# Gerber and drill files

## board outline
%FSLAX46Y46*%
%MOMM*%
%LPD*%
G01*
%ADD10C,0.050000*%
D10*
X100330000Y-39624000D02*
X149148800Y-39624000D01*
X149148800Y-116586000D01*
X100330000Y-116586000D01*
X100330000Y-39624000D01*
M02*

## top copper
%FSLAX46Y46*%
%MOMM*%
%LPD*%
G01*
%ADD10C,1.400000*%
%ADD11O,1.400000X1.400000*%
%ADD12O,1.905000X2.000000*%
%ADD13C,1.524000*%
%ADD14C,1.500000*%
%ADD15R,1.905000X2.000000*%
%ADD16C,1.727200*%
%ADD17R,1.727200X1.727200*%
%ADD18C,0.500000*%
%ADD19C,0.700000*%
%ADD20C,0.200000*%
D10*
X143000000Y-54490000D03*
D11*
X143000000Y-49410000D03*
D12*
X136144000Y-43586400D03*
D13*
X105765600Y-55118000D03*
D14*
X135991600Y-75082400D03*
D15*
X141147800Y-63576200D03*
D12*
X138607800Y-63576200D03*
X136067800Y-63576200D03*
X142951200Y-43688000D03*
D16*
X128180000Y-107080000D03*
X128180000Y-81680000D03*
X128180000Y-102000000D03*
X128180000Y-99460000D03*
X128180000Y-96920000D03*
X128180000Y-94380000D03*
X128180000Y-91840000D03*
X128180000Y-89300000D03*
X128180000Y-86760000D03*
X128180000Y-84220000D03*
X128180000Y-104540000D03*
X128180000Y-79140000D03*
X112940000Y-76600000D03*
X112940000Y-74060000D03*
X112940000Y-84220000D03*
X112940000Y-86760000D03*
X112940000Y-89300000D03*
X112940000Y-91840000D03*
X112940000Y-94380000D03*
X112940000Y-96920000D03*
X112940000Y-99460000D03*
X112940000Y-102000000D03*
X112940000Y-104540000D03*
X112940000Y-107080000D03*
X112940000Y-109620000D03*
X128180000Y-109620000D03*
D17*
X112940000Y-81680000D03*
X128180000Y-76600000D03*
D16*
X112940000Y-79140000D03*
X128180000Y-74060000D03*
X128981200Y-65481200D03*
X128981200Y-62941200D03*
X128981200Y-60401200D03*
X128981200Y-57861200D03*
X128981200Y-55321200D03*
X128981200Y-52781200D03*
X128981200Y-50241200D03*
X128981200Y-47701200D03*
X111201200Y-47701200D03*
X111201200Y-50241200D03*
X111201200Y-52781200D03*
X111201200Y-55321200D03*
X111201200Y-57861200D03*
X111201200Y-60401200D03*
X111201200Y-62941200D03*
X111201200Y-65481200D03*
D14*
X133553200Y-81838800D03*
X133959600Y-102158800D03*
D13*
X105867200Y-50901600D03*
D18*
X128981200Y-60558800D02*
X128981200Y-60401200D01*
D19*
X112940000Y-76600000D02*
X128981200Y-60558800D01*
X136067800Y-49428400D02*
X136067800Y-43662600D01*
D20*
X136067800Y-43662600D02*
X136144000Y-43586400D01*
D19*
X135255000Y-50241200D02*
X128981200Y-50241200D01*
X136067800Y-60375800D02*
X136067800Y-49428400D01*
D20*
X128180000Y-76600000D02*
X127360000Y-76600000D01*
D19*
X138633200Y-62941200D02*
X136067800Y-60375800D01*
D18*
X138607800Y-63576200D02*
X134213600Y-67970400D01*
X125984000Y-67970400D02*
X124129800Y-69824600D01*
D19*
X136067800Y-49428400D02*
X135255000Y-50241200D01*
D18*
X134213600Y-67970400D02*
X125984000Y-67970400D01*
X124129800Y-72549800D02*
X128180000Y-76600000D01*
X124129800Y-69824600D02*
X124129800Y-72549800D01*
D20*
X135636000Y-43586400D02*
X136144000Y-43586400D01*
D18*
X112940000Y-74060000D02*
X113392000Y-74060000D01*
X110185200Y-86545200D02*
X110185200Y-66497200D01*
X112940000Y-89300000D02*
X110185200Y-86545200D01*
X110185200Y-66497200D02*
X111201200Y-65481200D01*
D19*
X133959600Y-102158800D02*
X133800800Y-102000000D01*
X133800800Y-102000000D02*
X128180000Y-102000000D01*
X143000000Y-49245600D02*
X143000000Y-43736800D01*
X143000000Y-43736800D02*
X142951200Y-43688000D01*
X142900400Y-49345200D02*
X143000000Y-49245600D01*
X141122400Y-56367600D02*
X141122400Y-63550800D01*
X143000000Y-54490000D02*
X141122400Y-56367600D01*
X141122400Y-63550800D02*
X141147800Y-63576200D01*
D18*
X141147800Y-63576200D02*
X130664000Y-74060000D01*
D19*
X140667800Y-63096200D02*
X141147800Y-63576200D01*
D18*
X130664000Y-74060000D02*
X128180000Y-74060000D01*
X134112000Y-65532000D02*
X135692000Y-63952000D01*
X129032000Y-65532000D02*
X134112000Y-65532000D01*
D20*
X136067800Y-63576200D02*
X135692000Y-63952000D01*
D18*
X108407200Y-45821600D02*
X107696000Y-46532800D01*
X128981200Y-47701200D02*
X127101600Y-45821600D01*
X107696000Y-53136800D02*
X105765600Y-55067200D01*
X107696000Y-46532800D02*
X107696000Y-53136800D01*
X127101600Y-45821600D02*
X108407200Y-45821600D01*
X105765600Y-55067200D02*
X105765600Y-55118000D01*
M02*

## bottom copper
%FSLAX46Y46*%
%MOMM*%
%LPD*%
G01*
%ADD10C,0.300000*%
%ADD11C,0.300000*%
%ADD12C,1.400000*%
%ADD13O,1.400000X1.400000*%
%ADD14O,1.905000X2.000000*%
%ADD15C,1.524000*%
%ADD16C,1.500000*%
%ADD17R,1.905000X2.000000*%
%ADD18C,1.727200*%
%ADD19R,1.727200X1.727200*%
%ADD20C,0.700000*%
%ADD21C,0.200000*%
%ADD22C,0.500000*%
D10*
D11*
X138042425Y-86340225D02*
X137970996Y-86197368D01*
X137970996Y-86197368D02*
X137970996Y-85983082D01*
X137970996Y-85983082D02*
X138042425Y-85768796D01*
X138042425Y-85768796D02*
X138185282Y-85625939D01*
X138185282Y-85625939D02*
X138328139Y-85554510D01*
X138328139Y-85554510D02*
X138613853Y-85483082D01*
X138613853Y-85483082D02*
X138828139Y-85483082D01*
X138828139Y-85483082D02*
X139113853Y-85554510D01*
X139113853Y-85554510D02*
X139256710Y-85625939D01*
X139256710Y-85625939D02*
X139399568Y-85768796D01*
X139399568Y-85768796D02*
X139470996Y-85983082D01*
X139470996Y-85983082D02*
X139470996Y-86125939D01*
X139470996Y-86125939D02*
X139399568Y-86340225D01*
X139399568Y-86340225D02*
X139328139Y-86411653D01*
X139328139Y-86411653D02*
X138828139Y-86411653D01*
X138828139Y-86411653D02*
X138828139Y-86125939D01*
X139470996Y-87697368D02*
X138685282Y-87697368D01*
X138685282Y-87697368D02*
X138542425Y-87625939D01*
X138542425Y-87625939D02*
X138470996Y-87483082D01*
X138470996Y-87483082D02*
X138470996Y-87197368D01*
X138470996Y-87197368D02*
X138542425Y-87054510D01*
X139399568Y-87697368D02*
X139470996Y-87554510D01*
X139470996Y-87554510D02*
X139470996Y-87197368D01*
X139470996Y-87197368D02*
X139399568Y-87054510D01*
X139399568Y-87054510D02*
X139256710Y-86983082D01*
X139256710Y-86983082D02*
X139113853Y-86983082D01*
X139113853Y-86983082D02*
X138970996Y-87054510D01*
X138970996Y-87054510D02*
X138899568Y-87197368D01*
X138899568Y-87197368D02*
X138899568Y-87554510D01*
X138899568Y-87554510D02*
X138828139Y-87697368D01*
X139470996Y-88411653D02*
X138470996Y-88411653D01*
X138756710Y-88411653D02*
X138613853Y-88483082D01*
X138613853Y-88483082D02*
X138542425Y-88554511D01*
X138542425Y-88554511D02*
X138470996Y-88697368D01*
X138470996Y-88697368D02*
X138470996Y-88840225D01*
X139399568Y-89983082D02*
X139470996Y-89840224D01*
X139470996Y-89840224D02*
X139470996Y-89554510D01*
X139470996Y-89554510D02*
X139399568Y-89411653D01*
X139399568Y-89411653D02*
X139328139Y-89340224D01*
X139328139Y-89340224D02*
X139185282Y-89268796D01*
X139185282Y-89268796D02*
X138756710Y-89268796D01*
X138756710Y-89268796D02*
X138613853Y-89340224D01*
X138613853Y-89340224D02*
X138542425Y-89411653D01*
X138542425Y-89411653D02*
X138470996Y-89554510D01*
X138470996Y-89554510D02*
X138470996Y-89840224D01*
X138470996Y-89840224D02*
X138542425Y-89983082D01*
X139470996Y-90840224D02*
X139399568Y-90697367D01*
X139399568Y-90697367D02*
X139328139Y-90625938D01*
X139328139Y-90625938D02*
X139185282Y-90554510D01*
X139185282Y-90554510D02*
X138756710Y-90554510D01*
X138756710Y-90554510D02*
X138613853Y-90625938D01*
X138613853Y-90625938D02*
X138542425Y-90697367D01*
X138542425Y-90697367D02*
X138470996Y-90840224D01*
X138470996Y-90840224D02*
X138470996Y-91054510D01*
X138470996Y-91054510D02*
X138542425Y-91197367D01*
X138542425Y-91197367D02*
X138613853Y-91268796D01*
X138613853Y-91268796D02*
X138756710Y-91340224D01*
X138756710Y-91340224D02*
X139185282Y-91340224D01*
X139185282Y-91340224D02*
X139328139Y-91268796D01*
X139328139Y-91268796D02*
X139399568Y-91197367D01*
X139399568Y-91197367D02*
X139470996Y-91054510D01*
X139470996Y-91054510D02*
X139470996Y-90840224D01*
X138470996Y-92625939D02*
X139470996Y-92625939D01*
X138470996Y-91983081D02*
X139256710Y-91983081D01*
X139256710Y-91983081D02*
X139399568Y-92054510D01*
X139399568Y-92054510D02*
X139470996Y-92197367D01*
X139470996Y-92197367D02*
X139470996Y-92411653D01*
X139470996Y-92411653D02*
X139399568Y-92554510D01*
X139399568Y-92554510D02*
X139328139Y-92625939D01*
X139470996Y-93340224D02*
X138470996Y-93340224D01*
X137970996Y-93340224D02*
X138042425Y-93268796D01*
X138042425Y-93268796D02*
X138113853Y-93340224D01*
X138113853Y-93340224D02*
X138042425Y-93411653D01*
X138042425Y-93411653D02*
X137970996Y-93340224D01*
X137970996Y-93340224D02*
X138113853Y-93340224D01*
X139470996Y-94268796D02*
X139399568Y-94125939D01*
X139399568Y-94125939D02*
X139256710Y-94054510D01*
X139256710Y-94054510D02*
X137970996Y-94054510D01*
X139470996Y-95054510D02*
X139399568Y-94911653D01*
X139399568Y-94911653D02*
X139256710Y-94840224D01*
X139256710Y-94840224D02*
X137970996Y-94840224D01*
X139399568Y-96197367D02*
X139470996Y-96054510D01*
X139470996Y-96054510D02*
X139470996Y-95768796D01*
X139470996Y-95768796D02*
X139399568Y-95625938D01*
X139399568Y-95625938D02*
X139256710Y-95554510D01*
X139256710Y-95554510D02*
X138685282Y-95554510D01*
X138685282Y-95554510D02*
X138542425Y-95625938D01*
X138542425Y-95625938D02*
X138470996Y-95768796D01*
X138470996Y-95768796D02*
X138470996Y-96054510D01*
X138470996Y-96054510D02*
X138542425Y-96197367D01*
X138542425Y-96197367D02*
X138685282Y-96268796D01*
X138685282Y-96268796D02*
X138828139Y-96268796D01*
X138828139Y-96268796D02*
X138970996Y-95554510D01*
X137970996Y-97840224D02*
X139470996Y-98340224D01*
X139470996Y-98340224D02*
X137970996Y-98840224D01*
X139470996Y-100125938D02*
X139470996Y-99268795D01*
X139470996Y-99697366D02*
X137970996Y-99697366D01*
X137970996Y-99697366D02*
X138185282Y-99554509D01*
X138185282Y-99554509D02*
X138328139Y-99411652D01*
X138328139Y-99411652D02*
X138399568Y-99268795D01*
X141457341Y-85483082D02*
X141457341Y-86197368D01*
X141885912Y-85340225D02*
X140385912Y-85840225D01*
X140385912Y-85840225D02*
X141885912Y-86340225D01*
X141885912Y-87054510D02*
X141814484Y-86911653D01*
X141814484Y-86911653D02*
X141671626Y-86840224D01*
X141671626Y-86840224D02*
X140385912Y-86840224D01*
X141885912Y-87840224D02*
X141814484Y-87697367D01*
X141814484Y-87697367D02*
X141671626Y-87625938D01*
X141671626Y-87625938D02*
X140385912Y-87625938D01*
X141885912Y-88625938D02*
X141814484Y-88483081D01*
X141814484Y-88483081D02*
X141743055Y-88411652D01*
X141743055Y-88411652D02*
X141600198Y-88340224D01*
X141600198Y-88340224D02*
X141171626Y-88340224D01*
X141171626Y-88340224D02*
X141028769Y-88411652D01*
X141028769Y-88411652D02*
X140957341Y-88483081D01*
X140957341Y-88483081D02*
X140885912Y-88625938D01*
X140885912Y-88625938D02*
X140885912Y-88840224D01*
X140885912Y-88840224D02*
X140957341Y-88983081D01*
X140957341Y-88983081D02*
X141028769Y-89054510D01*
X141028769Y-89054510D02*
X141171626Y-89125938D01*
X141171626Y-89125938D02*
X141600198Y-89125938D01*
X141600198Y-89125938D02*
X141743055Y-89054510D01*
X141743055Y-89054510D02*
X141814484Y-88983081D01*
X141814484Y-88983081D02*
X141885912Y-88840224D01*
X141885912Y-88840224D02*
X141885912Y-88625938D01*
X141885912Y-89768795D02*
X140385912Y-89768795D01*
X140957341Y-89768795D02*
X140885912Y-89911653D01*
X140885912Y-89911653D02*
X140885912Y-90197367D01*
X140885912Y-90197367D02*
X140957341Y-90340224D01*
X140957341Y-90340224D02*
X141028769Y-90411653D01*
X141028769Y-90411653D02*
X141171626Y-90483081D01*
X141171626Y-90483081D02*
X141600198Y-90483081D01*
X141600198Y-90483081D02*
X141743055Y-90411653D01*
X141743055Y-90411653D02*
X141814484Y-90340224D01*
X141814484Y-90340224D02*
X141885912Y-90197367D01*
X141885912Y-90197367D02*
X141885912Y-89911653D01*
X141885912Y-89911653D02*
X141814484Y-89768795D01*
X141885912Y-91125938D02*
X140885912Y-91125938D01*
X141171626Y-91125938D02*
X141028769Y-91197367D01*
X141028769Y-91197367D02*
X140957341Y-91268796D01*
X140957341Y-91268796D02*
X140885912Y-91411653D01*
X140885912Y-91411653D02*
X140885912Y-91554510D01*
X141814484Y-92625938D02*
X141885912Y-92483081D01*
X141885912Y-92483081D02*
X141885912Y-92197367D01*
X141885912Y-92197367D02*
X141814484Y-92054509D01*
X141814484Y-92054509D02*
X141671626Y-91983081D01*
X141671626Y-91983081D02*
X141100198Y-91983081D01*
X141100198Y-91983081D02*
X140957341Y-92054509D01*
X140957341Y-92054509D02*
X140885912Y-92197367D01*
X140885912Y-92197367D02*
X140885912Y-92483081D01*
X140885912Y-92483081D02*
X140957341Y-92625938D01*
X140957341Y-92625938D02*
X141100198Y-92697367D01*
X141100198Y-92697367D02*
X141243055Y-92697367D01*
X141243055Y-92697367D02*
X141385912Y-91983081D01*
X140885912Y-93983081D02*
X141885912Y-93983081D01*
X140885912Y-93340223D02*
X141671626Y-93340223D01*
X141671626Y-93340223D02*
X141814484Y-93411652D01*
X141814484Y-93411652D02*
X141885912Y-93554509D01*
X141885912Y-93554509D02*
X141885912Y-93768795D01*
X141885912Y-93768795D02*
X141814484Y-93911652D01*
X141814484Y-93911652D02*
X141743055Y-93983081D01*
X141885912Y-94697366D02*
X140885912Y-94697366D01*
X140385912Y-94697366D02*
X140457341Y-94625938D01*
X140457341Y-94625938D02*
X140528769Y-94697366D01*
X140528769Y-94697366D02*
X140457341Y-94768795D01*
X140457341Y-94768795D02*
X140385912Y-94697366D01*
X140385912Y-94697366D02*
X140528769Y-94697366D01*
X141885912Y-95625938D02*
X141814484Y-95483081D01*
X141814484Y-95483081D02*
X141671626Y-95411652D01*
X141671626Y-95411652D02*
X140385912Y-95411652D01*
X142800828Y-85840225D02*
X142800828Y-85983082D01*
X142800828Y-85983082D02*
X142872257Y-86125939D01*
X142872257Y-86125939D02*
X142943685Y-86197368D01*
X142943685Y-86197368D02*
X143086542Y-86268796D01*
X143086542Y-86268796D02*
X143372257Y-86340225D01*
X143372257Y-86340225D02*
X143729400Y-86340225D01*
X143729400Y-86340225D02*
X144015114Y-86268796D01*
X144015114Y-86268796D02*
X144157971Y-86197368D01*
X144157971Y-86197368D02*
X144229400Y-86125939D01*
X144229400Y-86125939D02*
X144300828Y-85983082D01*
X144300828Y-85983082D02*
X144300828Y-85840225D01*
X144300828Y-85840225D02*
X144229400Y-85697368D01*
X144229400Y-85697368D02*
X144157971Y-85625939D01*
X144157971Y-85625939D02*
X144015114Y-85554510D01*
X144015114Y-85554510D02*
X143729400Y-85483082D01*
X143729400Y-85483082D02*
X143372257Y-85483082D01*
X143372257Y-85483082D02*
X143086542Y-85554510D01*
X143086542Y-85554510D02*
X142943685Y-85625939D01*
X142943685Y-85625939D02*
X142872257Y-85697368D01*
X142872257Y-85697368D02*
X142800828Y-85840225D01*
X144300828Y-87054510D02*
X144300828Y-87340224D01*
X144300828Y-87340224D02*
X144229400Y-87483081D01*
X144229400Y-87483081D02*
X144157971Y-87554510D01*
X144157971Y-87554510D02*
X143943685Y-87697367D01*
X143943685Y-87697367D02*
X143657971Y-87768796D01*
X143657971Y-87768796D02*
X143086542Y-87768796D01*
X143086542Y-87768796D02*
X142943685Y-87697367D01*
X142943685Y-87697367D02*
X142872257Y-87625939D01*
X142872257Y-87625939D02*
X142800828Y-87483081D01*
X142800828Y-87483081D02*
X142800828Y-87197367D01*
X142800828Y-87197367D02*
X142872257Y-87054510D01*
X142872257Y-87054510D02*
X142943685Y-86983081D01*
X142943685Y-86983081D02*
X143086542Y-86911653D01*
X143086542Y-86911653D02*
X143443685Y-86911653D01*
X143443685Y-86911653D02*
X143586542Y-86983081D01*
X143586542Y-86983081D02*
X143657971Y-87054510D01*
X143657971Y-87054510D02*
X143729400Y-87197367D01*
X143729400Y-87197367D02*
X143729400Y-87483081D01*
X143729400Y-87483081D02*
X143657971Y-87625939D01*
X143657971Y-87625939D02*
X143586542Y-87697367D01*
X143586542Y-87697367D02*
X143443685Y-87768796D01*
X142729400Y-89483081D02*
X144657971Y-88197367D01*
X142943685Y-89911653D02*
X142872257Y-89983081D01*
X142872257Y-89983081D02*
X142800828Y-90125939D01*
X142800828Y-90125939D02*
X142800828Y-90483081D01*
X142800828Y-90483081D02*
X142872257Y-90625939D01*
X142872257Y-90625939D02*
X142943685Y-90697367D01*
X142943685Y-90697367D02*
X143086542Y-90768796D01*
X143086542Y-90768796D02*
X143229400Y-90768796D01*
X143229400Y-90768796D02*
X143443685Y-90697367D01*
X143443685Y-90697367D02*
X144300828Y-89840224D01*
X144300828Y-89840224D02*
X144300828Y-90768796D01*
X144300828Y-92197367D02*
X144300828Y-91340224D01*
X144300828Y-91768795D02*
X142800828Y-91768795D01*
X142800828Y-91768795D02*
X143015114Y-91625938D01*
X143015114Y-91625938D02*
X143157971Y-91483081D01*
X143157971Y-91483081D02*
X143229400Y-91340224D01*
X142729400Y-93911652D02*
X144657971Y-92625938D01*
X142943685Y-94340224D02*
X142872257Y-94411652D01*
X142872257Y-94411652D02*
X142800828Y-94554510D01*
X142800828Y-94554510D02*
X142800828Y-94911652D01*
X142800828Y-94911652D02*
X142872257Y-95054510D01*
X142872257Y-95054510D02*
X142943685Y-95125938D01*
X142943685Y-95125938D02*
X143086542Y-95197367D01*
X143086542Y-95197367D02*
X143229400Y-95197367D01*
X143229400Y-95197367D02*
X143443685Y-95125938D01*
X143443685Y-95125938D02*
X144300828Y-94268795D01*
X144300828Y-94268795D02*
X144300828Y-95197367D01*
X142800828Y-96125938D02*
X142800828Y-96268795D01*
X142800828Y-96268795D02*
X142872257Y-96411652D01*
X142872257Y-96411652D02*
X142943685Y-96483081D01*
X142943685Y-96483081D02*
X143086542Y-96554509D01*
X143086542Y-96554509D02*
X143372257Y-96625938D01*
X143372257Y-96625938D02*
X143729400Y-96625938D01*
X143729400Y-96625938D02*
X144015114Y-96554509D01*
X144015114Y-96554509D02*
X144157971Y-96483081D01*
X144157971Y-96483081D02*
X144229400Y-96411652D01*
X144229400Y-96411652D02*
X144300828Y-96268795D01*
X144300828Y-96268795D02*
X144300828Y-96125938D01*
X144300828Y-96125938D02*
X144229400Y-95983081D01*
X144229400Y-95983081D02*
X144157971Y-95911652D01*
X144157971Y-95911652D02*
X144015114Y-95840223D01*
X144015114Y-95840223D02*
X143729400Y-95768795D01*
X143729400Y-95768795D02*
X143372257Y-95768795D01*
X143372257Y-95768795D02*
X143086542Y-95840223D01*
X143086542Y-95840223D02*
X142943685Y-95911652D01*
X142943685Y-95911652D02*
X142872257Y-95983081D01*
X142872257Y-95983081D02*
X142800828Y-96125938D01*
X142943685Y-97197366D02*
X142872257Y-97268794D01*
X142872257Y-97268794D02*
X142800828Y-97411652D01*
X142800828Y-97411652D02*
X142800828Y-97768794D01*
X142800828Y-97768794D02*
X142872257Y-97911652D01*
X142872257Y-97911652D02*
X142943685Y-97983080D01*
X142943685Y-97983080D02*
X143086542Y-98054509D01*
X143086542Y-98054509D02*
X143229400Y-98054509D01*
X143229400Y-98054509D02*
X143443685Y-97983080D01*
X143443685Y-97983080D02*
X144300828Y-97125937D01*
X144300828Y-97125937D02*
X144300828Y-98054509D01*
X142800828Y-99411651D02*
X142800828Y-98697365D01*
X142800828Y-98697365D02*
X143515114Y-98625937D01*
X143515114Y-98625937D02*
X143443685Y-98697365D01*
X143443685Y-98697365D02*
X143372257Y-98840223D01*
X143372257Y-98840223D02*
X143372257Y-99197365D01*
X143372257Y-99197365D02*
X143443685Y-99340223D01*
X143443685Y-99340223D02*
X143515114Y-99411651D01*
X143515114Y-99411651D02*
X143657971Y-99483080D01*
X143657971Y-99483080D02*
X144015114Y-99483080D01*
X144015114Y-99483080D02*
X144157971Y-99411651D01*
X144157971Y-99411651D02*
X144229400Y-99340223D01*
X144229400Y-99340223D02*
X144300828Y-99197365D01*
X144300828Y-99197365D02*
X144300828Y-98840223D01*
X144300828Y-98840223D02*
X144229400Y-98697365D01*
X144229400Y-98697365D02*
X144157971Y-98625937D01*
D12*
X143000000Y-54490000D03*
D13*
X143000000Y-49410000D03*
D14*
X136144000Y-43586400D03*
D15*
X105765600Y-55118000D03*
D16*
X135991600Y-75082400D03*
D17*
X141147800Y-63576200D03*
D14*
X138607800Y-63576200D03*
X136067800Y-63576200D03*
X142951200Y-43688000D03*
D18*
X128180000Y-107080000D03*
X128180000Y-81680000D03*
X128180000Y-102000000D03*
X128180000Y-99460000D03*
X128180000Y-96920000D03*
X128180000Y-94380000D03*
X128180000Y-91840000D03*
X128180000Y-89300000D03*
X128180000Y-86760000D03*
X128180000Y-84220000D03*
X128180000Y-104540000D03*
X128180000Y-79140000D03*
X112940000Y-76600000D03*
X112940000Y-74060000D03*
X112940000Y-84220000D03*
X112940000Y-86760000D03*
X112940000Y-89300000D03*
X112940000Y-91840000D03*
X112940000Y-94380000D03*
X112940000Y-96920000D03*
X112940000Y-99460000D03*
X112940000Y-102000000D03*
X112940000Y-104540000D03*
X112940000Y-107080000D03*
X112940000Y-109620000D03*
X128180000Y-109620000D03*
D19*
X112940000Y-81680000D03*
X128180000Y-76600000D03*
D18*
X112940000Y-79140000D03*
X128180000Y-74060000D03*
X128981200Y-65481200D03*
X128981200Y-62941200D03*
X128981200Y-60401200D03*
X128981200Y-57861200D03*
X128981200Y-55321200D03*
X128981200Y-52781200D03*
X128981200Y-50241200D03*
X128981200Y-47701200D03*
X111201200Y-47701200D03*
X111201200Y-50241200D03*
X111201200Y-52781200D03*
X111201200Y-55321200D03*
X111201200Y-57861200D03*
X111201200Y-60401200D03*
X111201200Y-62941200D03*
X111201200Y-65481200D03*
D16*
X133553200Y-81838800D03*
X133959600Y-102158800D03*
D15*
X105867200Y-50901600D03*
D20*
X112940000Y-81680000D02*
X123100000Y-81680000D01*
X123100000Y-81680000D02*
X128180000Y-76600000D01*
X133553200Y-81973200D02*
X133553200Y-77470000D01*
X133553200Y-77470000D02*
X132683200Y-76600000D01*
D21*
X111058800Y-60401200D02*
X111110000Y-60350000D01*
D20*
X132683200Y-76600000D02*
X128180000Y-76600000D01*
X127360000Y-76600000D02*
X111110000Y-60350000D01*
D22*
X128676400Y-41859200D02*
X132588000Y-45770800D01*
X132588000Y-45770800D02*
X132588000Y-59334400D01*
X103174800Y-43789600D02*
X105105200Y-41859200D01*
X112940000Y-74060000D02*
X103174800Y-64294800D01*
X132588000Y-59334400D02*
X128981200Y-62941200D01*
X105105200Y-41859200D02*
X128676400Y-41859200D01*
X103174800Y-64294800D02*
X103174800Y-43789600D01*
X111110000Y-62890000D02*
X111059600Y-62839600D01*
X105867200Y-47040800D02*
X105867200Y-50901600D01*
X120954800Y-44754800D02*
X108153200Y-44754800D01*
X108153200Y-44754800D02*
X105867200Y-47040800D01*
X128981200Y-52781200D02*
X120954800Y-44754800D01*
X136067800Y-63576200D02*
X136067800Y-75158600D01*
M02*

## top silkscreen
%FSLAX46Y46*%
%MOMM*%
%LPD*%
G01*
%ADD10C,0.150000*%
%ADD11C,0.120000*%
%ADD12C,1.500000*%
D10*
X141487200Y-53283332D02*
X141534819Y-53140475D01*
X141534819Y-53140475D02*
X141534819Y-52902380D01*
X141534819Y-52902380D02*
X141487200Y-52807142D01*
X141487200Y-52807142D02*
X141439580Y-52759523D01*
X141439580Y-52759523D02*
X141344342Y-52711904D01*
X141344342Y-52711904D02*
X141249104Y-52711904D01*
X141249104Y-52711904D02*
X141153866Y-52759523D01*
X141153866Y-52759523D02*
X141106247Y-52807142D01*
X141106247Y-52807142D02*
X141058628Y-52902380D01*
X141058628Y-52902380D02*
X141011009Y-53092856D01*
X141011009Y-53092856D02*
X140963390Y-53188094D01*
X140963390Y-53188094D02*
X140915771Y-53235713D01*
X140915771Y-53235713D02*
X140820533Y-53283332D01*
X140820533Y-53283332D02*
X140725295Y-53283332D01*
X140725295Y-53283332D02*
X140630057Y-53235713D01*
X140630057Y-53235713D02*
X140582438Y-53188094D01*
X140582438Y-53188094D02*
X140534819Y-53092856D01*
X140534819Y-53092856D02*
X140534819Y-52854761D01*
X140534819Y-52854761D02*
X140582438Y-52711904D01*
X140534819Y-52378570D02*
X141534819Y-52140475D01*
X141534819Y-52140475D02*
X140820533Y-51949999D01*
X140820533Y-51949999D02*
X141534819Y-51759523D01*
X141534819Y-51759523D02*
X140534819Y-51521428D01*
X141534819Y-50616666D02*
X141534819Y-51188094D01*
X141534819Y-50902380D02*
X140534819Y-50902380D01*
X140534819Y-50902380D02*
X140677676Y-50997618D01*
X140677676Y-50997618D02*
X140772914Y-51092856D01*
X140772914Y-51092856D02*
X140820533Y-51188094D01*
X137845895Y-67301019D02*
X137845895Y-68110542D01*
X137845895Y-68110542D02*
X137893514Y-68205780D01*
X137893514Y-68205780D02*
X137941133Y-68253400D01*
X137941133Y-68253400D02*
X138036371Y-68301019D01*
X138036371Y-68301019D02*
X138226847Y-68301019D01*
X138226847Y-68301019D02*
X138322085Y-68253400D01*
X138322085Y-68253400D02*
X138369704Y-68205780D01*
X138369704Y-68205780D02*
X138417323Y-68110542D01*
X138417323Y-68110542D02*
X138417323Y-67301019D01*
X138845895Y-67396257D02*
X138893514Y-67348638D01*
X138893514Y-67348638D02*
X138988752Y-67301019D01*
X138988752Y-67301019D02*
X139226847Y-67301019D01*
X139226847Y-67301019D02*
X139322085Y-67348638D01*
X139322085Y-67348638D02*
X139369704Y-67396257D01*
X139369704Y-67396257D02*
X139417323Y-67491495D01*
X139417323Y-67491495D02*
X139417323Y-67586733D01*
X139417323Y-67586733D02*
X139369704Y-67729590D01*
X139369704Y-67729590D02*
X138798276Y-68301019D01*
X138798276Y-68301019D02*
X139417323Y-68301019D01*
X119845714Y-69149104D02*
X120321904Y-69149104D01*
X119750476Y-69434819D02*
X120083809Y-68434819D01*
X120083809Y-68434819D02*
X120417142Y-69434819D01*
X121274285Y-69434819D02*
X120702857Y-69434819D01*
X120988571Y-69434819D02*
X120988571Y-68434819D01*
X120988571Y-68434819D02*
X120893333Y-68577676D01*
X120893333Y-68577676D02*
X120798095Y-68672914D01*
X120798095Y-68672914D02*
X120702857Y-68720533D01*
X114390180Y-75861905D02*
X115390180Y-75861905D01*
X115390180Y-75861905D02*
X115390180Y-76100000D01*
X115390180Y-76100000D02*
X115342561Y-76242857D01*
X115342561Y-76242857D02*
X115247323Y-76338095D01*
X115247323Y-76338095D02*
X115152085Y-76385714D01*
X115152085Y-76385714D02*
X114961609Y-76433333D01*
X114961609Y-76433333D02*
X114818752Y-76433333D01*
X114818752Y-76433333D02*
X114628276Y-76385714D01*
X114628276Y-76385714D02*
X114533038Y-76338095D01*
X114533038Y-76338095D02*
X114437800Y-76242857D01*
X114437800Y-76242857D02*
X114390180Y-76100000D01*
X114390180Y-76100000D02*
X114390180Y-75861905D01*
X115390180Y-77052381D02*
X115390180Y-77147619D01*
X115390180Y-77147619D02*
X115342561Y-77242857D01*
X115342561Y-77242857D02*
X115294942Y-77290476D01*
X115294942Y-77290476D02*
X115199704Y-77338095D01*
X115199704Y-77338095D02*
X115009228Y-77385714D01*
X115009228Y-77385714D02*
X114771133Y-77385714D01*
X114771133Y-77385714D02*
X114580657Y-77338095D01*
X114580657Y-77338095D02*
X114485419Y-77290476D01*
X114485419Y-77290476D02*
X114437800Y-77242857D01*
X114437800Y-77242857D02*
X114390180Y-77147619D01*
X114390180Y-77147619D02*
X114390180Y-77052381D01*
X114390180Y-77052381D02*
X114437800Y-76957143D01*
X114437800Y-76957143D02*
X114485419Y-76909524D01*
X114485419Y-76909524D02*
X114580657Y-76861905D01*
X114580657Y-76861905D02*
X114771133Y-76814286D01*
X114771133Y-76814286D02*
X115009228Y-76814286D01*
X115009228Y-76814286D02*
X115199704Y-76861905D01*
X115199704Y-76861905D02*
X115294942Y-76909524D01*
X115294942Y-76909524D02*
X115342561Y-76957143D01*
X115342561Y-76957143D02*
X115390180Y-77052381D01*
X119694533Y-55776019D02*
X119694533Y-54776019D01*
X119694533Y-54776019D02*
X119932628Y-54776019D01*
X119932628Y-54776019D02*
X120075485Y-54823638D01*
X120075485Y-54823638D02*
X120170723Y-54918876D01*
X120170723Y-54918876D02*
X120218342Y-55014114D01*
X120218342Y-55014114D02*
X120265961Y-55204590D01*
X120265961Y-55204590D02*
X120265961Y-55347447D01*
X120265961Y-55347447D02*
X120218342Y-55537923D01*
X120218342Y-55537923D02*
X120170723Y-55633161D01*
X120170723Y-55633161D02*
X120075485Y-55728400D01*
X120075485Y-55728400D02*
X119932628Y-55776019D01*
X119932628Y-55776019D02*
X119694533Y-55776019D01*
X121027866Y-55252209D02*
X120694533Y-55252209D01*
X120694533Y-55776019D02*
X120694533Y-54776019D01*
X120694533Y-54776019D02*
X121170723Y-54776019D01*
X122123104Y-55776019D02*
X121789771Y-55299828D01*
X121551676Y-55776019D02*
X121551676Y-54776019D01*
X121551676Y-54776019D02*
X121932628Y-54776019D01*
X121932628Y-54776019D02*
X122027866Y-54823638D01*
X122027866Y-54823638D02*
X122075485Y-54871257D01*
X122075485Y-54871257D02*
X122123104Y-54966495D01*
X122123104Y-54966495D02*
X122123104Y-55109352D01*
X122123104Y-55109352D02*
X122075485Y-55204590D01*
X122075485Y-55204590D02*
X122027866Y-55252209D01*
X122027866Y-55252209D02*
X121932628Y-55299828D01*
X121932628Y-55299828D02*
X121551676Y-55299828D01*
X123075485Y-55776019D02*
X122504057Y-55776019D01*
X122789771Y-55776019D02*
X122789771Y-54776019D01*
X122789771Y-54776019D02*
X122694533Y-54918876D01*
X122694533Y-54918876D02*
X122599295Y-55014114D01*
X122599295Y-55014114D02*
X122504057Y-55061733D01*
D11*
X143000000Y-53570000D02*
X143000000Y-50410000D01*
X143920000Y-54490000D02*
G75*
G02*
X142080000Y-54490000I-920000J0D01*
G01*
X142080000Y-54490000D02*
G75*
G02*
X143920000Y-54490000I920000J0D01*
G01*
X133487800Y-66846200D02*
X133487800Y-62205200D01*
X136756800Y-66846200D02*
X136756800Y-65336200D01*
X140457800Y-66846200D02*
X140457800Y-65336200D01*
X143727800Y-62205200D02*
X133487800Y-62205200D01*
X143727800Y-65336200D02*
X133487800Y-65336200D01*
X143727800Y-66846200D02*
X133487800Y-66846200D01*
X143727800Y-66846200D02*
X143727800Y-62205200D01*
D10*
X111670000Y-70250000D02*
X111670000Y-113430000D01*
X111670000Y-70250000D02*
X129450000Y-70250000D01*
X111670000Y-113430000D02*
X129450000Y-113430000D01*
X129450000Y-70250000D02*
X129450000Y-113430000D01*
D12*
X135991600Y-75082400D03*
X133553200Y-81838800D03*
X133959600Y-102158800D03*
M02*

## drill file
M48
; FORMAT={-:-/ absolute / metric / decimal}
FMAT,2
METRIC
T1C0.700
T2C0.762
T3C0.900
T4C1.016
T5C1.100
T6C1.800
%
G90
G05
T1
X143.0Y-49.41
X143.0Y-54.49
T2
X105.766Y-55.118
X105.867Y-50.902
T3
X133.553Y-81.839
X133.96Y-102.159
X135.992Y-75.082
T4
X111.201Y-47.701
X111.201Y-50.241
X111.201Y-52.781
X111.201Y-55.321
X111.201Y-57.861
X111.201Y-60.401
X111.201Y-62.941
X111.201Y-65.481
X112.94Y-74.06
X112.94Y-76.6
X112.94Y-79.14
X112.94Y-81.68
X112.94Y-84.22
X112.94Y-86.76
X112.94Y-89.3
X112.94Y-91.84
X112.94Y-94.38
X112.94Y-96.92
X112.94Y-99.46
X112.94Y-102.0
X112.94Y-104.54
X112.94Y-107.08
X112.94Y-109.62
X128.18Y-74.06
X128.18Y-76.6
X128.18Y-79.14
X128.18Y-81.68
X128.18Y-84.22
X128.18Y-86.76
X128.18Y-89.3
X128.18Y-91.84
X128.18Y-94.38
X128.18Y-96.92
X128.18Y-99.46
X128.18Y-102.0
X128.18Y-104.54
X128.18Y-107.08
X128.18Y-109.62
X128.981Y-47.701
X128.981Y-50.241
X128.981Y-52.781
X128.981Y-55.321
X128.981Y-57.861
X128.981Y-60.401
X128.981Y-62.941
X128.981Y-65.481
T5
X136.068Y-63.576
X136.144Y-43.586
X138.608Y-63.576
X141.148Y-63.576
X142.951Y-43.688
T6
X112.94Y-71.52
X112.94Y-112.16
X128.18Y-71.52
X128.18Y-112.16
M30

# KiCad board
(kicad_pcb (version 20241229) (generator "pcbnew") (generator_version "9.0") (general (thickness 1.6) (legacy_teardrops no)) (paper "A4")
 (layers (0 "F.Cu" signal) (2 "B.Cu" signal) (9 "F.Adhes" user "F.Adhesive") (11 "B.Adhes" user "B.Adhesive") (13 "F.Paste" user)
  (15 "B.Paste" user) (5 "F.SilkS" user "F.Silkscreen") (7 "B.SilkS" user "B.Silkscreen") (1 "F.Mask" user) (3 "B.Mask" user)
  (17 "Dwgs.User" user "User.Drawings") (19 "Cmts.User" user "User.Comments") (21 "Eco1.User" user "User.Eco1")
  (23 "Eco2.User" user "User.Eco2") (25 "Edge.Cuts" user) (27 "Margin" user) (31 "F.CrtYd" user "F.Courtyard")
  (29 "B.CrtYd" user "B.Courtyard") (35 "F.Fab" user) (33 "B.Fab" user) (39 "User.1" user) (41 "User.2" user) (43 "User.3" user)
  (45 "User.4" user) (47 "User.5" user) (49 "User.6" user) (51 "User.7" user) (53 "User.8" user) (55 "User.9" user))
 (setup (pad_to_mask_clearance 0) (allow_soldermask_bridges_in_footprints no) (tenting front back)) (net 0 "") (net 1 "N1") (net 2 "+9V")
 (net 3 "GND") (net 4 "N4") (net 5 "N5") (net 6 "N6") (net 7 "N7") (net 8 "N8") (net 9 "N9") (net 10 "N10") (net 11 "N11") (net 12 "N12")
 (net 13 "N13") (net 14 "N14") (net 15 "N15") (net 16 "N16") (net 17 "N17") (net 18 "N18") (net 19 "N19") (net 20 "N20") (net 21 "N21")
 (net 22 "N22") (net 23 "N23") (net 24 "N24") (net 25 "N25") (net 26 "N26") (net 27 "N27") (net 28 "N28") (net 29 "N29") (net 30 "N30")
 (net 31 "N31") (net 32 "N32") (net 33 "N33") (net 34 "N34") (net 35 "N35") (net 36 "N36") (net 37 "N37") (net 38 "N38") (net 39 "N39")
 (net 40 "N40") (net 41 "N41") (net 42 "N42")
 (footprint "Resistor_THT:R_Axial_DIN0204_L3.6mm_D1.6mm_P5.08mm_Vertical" (layer "F.Cu") (at 143 54.49 90)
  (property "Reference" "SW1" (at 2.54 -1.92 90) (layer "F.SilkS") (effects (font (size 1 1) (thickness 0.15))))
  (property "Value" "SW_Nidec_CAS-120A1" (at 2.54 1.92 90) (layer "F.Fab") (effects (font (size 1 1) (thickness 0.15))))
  (fp_line (start 0.92 0) (end 4.08 0) (stroke (width 0.12) (type solid)) (layer "F.SilkS"))
  (fp_circle (center 0 0) (end 0.92 0) (stroke (width 0.12) (type solid)) (fill no) (layer "F.SilkS"))
  (pad "1" thru_hole circle (at 0 0 90) (size 1.4 1.4) (drill 0.7) (layers "*.Cu" "*.Mask") (remove_unused_layers no) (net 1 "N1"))
  (pad "2" thru_hole oval (at 5.08 0 90) (size 1.4 1.4) (drill 0.7) (layers "*.Cu" "*.Mask") (remove_unused_layers no) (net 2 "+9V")))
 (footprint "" (layer "F.Cu") (at 136.144 43.5864)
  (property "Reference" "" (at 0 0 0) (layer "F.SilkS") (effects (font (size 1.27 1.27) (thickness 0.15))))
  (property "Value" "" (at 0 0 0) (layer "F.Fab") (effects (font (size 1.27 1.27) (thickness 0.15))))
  (pad "3" thru_hole oval (at 0 0 180) (size 1.905 2) (drill 1.1) (layers "*.Cu" "*.Mask") (remove_unused_layers no) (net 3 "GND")))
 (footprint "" (layer "F.Cu") (at 105.7656 55.118)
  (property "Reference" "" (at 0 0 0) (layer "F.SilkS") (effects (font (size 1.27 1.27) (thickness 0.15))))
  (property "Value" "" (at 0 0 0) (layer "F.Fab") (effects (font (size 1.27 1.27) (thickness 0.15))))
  (pad "8" thru_hole circle (at 0 0) (size 1.524 1.524) (drill 0.762) (layers "*.Cu" "*.Mask") (remove_unused_layers no) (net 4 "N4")))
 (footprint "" (layer "F.Cu") (at 135.9916 75.0824)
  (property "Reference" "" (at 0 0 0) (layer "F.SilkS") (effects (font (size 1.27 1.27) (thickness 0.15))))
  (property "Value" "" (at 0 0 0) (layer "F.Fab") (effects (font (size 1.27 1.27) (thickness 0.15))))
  (pad "3" thru_hole circle (at 0 0 90) (size 1.5 1.5) (drill 0.9) (layers "*.Cu" "*.Mask" "F.SilkS") (remove_unused_layers no) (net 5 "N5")))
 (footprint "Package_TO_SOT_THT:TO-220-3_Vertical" (layer "F.Cu") (at 141.1478 63.5762 180)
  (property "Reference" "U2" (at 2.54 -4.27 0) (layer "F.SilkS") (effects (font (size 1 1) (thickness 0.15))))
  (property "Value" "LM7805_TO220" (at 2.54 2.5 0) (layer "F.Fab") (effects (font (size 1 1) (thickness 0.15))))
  (fp_line (start 7.66 -3.27) (end 7.66 1.371) (stroke (width 0.12) (type solid)) (layer "F.SilkS"))
  (fp_line (start 4.391 -3.27) (end 4.391 -1.76) (stroke (width 0.12) (type solid)) (layer "F.SilkS"))
  (fp_line (start 0.69 -3.27) (end 0.69 -1.76) (stroke (width 0.12) (type solid)) (layer "F.SilkS"))
  (fp_line (start -2.58 1.371) (end 7.66 1.371) (stroke (width 0.12) (type solid)) (layer "F.SilkS"))
  (fp_line (start -2.58 -1.76) (end 7.66 -1.76) (stroke (width 0.12) (type solid)) (layer "F.SilkS"))
  (fp_line (start -2.58 -3.27) (end 7.66 -3.27) (stroke (width 0.12) (type solid)) (layer "F.SilkS"))
  (fp_line (start -2.58 -3.27) (end -2.58 1.371) (stroke (width 0.12) (type solid)) (layer "F.SilkS"))
  (pad "1" thru_hole rect (at 0 0 180) (size 1.905 2) (drill 1.1) (layers "*.Cu" "*.Mask") (remove_unused_layers no) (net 1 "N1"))
  (pad "2" thru_hole oval (at 2.54 0 180) (size 1.905 2) (drill 1.1) (layers "*.Cu" "*.Mask") (remove_unused_layers no) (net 3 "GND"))
  (pad "3" thru_hole oval (at 5.08 0 180) (size 1.905 2) (drill 1.1) (layers "*.Cu" "*.Mask") (remove_unused_layers no) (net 5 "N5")))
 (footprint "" (layer "F.Cu") (at 142.9512 43.688)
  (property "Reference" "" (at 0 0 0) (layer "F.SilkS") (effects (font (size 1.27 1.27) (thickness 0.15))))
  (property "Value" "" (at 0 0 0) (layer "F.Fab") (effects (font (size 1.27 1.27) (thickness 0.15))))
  (pad "3" thru_hole oval (at 0 0 180) (size 1.905 2) (drill 1.1) (layers "*.Cu" "*.Mask") (remove_unused_layers no) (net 2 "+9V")))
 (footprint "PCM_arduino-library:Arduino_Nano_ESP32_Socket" (layer "F.Cu") (at 120.56 113.43)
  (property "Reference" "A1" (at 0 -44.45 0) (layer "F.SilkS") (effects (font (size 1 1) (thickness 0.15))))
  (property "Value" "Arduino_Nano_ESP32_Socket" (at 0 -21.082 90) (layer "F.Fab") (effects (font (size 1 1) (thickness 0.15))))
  (fp_line (start -8.89 -43.18) (end -8.89 0) (stroke (width 0.15) (type solid)) (layer "F.SilkS"))
  (fp_line (start -8.89 -43.18) (end 8.89 -43.18) (stroke (width 0.15) (type solid)) (layer "F.SilkS"))
  (fp_line (start -8.89 0) (end 8.89 0) (stroke (width 0.15) (type solid)) (layer "F.SilkS"))
  (fp_line (start 8.89 -43.18) (end 8.89 0) (stroke (width 0.15) (type solid)) (layer "F.SilkS"))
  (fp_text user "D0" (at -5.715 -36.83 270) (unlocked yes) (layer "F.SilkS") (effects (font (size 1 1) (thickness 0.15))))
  (pad "" np_thru_hole circle (at -7.62 -41.91) (size 1.8 1.8) (drill 1.8) (layers "*.Cu" "*.Mask"))
  (pad "" np_thru_hole circle (at -7.62 -1.27) (size 1.8 1.8) (drill 1.8) (layers "*.Cu" "*.Mask"))
  (pad "" np_thru_hole circle (at 7.62 -41.91) (size 1.8 1.8) (drill 1.8) (layers "*.Cu" "*.Mask"))
  (pad "" np_thru_hole circle (at 7.62 -1.27) (size 1.8 1.8) (drill 1.8) (layers "*.Cu" "*.Mask"))
  (pad "3V3" thru_hole circle (at 7.62 -6.35) (size 1.7272 1.7272) (drill 1.016) (layers "*.Cu" "*.Mask") (remove_unused_layers no)
   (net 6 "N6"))
  (pad "5V" thru_hole circle (at 7.62 -31.75) (size 1.7272 1.7272) (drill 1.016) (layers "*.Cu" "*.Mask") (remove_unused_layers no)
   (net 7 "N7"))
  (pad "A0" thru_hole circle (at 7.62 -11.43) (size 1.7272 1.7272) (drill 1.016) (layers "*.Cu" "*.Mask") (remove_unused_layers no)
   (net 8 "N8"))
  (pad "A1" thru_hole circle (at 7.62 -13.97) (size 1.7272 1.7272) (drill 1.016) (layers "*.Cu" "*.Mask") (remove_unused_layers no)
   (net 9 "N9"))
  (pad "A2" thru_hole circle (at 7.62 -16.51) (size 1.7272 1.7272) (drill 1.016) (layers "*.Cu" "*.Mask") (remove_unused_layers no)
   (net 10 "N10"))
  (pad "A3" thru_hole circle (at 7.62 -19.05) (size 1.7272 1.7272) (drill 1.016) (layers "*.Cu" "*.Mask") (remove_unused_layers no)
   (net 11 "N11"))
  (pad "A4" thru_hole circle (at 7.62 -21.59) (size 1.7272 1.7272) (drill 1.016) (layers "*.Cu" "*.Mask") (remove_unused_layers no)
   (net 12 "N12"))
  (pad "A5" thru_hole circle (at 7.62 -24.13) (size 1.7272 1.7272) (drill 1.016) (layers "*.Cu" "*.Mask") (remove_unused_layers no)
   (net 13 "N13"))
  (pad "A6" thru_hole circle (at 7.62 -26.67) (size 1.7272 1.7272) (drill 1.016) (layers "*.Cu" "*.Mask") (remove_unused_layers no)
   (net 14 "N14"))
  (pad "A7" thru_hole circle (at 7.62 -29.21) (size 1.7272 1.7272) (drill 1.016) (layers "*.Cu" "*.Mask") (remove_unused_layers no)
   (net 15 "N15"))
  (pad "B0" thru_hole circle (at 7.62 -8.89) (size 1.7272 1.7272) (drill 1.016) (layers "*.Cu" "*.Mask") (remove_unused_layers no)
   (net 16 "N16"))
  (pad "B1" thru_hole circle (at 7.62 -34.29) (size 1.7272 1.7272) (drill 1.016) (layers "*.Cu" "*.Mask") (remove_unused_layers no)
   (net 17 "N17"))
  (pad "D0" thru_hole circle (at -7.62 -36.83) (size 1.7272 1.7272) (drill 1.016) (layers "*.Cu" "*.Mask") (remove_unused_layers no)
   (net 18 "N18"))
  (pad "D1" thru_hole circle (at -7.62 -39.37) (size 1.7272 1.7272) (drill 1.016) (layers "*.Cu" "*.Mask") (remove_unused_layers no)
   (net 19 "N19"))
  (pad "D2" thru_hole circle (at -7.62 -29.21) (size 1.7272 1.7272) (drill 1.016) (layers "*.Cu" "*.Mask") (remove_unused_layers no)
   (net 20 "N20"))
  (pad "D3" thru_hole circle (at -7.62 -26.67) (size 1.7272 1.7272) (drill 1.016) (layers "*.Cu" "*.Mask") (remove_unused_layers no)
   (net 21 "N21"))
  (pad "D4" thru_hole circle (at -7.62 -24.13) (size 1.7272 1.7272) (drill 1.016) (layers "*.Cu" "*.Mask") (remove_unused_layers no)
   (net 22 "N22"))
  (pad "D5" thru_hole circle (at -7.62 -21.59) (size 1.7272 1.7272) (drill 1.016) (layers "*.Cu" "*.Mask") (remove_unused_layers no)
   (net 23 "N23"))
  (pad "D6" thru_hole circle (at -7.62 -19.05) (size 1.7272 1.7272) (drill 1.016) (layers "*.Cu" "*.Mask") (remove_unused_layers no)
   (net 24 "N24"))
  (pad "D7" thru_hole circle (at -7.62 -16.51) (size 1.7272 1.7272) (drill 1.016) (layers "*.Cu" "*.Mask") (remove_unused_layers no)
   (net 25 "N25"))
  (pad "D8" thru_hole circle (at -7.62 -13.97) (size 1.7272 1.7272) (drill 1.016) (layers "*.Cu" "*.Mask") (remove_unused_layers no)
   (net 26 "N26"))
  (pad "D9" thru_hole circle (at -7.62 -11.43) (size 1.7272 1.7272) (drill 1.016) (layers "*.Cu" "*.Mask") (remove_unused_layers no)
   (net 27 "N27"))
  (pad "D10" thru_hole circle (at -7.62 -8.89) (size 1.7272 1.7272) (drill 1.016) (layers "*.Cu" "*.Mask") (remove_unused_layers no)
   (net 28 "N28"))
  (pad "D11" thru_hole circle (at -7.62 -6.35) (size 1.7272 1.7272) (drill 1.016) (layers "*.Cu" "*.Mask") (remove_unused_layers no)
   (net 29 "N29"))
  (pad "D12" thru_hole circle (at -7.62 -3.81) (size 1.7272 1.7272) (drill 1.016) (layers "*.Cu" "*.Mask") (remove_unused_layers no)
   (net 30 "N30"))
  (pad "D13" thru_hole circle (at 7.62 -3.81) (size 1.7272 1.7272) (drill 1.016) (layers "*.Cu" "*.Mask") (remove_unused_layers no)
   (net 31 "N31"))
  (pad "GND1" thru_hole rect (at -7.62 -31.75) (size 1.7272 1.7272) (drill 1.016) (layers "*.Cu" "*.Mask") (remove_unused_layers no)
   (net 3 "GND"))
  (pad "GND2" thru_hole rect (at 7.62 -36.83) (size 1.7272 1.7272) (drill 1.016) (layers "*.Cu" "*.Mask") (remove_unused_layers no)
   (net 3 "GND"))
  (pad "RST" thru_hole circle (at -7.62 -34.29) (size 1.7272 1.7272) (drill 1.016) (layers "*.Cu" "*.Mask") (remove_unused_layers no)
   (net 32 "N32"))
  (pad "VIN" thru_hole circle (at 7.62 -39.37) (size 1.7272 1.7272) (drill 1.016) (layers "*.Cu" "*.Mask") (remove_unused_layers no)
   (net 1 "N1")))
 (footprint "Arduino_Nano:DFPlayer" (layer "F.Cu") (at 121.3612 65.4812 180)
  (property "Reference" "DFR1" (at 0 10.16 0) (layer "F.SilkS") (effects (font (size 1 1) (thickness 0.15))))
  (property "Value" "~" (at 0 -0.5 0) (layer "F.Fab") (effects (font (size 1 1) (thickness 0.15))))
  (pad "1" thru_hole circle (at -7.62 0 180) (size 1.7272 1.7272) (drill 1.016) (layers "*.Cu" "*.Mask") (remove_unused_layers no)
   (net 5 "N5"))
  (pad "2" thru_hole circle (at -7.62 2.54 180) (size 1.7272 1.7272) (drill 1.016) (layers "*.Cu" "*.Mask") (remove_unused_layers no)
   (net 19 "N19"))
  (pad "3" thru_hole circle (at -7.62 5.08 180) (size 1.7272 1.7272) (drill 1.016) (layers "*.Cu" "*.Mask") (remove_unused_layers no)
   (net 18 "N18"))
  (pad "4" thru_hole circle (at -7.62 7.62 180) (size 1.7272 1.7272) (drill 1.016) (layers "*.Cu" "*.Mask") (remove_unused_layers no)
   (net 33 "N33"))
  (pad "5" thru_hole circle (at -7.62 10.16 180) (size 1.7272 1.7272) (drill 1.016) (layers "*.Cu" "*.Mask") (remove_unused_layers no)
   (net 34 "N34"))
  (pad "6" thru_hole circle (at -7.62 12.7 180) (size 1.7272 1.7272) (drill 1.016) (layers "*.Cu" "*.Mask") (remove_unused_layers no)
   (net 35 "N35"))
  (pad "7" thru_hole circle (at -7.62 15.24 180) (size 1.7272 1.7272) (drill 1.016) (layers "*.Cu" "*.Mask") (remove_unused_layers no)
   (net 3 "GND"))
  (pad "8" thru_hole circle (at -7.62 17.78 180) (size 1.7272 1.7272) (drill 1.016) (layers "*.Cu" "*.Mask") (remove_unused_layers no)
   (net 4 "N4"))
  (pad "9" thru_hole circle (at 10.16 17.78 180) (size 1.7272 1.7272) (drill 1.016) (layers "*.Cu" "*.Mask") (remove_unused_layers no)
   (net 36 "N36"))
  (pad "10" thru_hole circle (at 10.16 15.24 180) (size 1.7272 1.7272) (drill 1.016) (layers "*.Cu" "*.Mask") (remove_unused_layers no)
   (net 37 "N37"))
  (pad "11" thru_hole circle (at 10.16 12.7 180) (size 1.7272 1.7272) (drill 1.016) (layers "*.Cu" "*.Mask") (remove_unused_layers no)
   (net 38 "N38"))
  (pad "12" thru_hole circle (at 10.16 10.16 180) (size 1.7272 1.7272) (drill 1.016) (layers "*.Cu" "*.Mask") (remove_unused_layers no)
   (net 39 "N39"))
  (pad "13" thru_hole circle (at 10.16 7.62 180) (size 1.7272 1.7272) (drill 1.016) (layers "*.Cu" "*.Mask") (remove_unused_layers no)
   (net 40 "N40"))
  (pad "14" thru_hole circle (at 10.16 5.08 180) (size 1.7272 1.7272) (drill 1.016) (layers "*.Cu" "*.Mask") (remove_unused_layers no)
   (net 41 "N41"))
  (pad "15" thru_hole circle (at 10.16 2.54 180) (size 1.7272 1.7272) (drill 1.016) (layers "*.Cu" "*.Mask") (remove_unused_layers no)
   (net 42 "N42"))
  (pad "16" thru_hole circle (at 10.16 0 180) (size 1.7272 1.7272) (drill 1.016) (layers "*.Cu" "*.Mask") (remove_unused_layers no)
   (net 22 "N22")))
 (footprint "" (layer "F.Cu") (at 133.5532 81.8388)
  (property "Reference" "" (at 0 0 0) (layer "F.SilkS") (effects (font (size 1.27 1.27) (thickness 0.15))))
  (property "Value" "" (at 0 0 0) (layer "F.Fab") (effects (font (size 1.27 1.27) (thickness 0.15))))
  (pad "1" thru_hole circle (at 0 0 90) (size 1.5 1.5) (drill 0.9) (layers "*.Cu" "*.Mask" "F.SilkS") (remove_unused_layers no)
   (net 3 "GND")))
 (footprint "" (layer "F.Cu") (at 133.9596 102.1588)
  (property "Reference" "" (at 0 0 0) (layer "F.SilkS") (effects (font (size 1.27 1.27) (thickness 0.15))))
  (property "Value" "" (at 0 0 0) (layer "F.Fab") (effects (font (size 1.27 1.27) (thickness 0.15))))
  (pad "2" thru_hole circle (at 0 0 90) (size 1.5 1.5) (drill 0.9) (layers "*.Cu" "*.Mask" "F.SilkS") (remove_unused_layers no) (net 8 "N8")))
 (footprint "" (layer "F.Cu") (at 105.8672 50.9016)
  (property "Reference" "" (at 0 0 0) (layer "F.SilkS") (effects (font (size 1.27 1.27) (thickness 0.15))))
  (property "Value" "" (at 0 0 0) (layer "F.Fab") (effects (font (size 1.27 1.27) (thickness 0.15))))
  (pad "6" thru_hole circle (at 0 0) (size 1.524 1.524) (drill 0.762) (layers "*.Cu" "*.Mask") (remove_unused_layers no) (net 35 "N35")))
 (gr_rect (start 100.33 39.624) (end 149.1488 116.586) (stroke (width 0.05) (type default)) (fill no) (layer "Edge.Cuts"))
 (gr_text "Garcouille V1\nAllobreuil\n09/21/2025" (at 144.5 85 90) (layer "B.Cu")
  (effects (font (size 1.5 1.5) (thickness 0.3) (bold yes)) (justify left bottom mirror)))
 (segment (start 128.9812 60.5588) (end 128.9812 60.4012) (width 0.5) (layer "F.Cu") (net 18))
 (segment (start 112.94 76.6) (end 128.9812 60.5588) (width 0.7) (layer "F.Cu") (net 18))
 (segment (start 136.0678 49.4284) (end 136.0678 43.6626) (width 0.7) (layer "F.Cu") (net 3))
 (segment (start 136.0678 43.6626) (end 136.144 43.5864) (width 0.2) (layer "F.Cu") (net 3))
 (segment (start 135.255 50.2412) (end 128.9812 50.2412) (width 0.7) (layer "F.Cu") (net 3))
 (segment (start 136.0678 60.3758) (end 136.0678 49.4284) (width 0.7) (layer "F.Cu") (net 3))
 (segment (start 128.18 76.6) (end 127.36 76.6) (width 0.2) (layer "F.Cu") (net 3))
 (segment (start 138.6332 62.9412) (end 136.0678 60.3758) (width 0.7) (layer "F.Cu") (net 3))
 (segment (start 138.6078 63.5762) (end 134.2136 67.9704) (width 0.5) (layer "F.Cu") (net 3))
 (segment (start 125.984 67.9704) (end 124.1298 69.8246) (width 0.5) (layer "F.Cu") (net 3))
 (segment (start 136.0678 49.4284) (end 135.255 50.2412) (width 0.7) (layer "F.Cu") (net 3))
 (segment (start 134.2136 67.9704) (end 125.984 67.9704) (width 0.5) (layer "F.Cu") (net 3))
 (segment (start 124.1298 72.5498) (end 128.18 76.6) (width 0.5) (layer "F.Cu") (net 3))
 (segment (start 124.1298 69.8246) (end 124.1298 72.5498) (width 0.5) (layer "F.Cu") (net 3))
 (segment (start 135.636 43.5864) (end 136.144 43.5864) (width 0.2) (layer "F.Cu") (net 3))
 (segment (start 112.94 81.68) (end 123.1 81.68) (width 0.7) (layer "B.Cu") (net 3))
 (segment (start 123.1 81.68) (end 128.18 76.6) (width 0.7) (layer "B.Cu") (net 3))
 (segment (start 133.5532 81.9732) (end 133.5532 77.47) (width 0.7) (layer "B.Cu") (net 3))
 (segment (start 133.5532 77.47) (end 132.6832 76.6) (width 0.7) (layer "B.Cu") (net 3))
 (segment (start 111.0588 60.4012) (end 111.11 60.35) (width 0.2) (layer "B.Cu") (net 3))
 (segment (start 132.6832 76.6) (end 128.18 76.6) (width 0.7) (layer "B.Cu") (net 3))
 (segment (start 127.36 76.6) (end 111.11 60.35) (width 0.7) (layer "B.Cu") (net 3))
 (segment (start 112.94 74.06) (end 113.392 74.06) (width 0.5) (layer "F.Cu") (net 19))
 (segment (start 128.6764 41.8592) (end 132.588 45.7708) (width 0.5) (layer "B.Cu") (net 19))
 (segment (start 132.588 45.7708) (end 132.588 59.3344) (width 0.5) (layer "B.Cu") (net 19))
 (segment (start 103.1748 43.7896) (end 105.1052 41.8592) (width 0.5) (layer "B.Cu") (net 19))
 (segment (start 112.94 74.06) (end 103.1748 64.2948) (width 0.5) (layer "B.Cu") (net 19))
 (segment (start 132.588 59.3344) (end 128.9812 62.9412) (width 0.5) (layer "B.Cu") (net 19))
 (segment (start 105.1052 41.8592) (end 128.6764 41.8592) (width 0.5) (layer "B.Cu") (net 19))
 (segment (start 103.1748 64.2948) (end 103.1748 43.7896) (width 0.5) (layer "B.Cu") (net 19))
 (segment (start 110.1852 86.5452) (end 110.1852 66.4972) (width 0.5) (layer "F.Cu") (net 22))
 (segment (start 112.94 89.3) (end 110.1852 86.5452) (width 0.5) (layer "F.Cu") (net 22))
 (segment (start 110.1852 66.4972) (end 111.2012 65.4812) (width 0.5) (layer "F.Cu") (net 22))
 (segment (start 111.11 62.89) (end 111.0596 62.8396) (width 0.5) (layer "B.Cu") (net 42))
 (segment (start 105.8672 47.0408) (end 105.8672 50.9016) (width 0.5) (layer "B.Cu") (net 35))
 (segment (start 120.9548 44.7548) (end 108.1532 44.7548) (width 0.5) (layer "B.Cu") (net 35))
 (segment (start 108.1532 44.7548) (end 105.8672 47.0408) (width 0.5) (layer "B.Cu") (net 35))
 (segment (start 128.9812 52.7812) (end 120.9548 44.7548) (width 0.5) (layer "B.Cu") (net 35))
 (segment (start 133.9596 102.1588) (end 133.8008 102) (width 0.7) (layer "F.Cu") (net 8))
 (segment (start 133.8008 102) (end 128.18 102) (width 0.7) (layer "F.Cu") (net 8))
 (segment (start 143 49.2456) (end 143 43.7368) (width 0.7) (layer "F.Cu") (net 2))
 (segment (start 143 43.7368) (end 142.9512 43.688) (width 0.7) (layer "F.Cu") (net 2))
 (segment (start 142.9004 49.3452) (end 143 49.2456) (width 0.7) (layer "F.Cu") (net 2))
 (segment (start 141.1224 56.3676) (end 141.1224 63.5508) (width 0.7) (layer "F.Cu") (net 1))
 (segment (start 143 54.49) (end 141.1224 56.3676) (width 0.7) (layer "F.Cu") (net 1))
 (segment (start 141.1224 63.5508) (end 141.1478 63.5762) (width 0.7) (layer "F.Cu") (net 1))
 (segment (start 141.1478 63.5762) (end 130.664 74.06) (width 0.5) (layer "F.Cu") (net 1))
 (segment (start 140.6678 63.0962) (end 141.1478 63.5762) (width 0.7) (layer "F.Cu") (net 1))
 (segment (start 130.664 74.06) (end 128.18 74.06) (width 0.5) (layer "F.Cu") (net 1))
 (segment (start 134.112 65.532) (end 135.692 63.952) (width 0.5) (layer "F.Cu") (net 5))
 (segment (start 129.032 65.532) (end 134.112 65.532) (width 0.5) (layer "F.Cu") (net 5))
 (segment (start 136.0678 63.5762) (end 135.692 63.952) (width 0.2) (layer "F.Cu") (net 5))
 (segment (start 136.0678 63.5762) (end 136.0678 75.1586) (width 0.5) (layer "B.Cu") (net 5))
 (segment (start 108.4072 45.8216) (end 107.696 46.5328) (width 0.5) (layer "F.Cu") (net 4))
 (segment (start 128.9812 47.7012) (end 127.1016 45.8216) (width 0.5) (layer "F.Cu") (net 4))
 (segment (start 107.696 53.1368) (end 105.7656 55.0672) (width 0.5) (layer "F.Cu") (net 4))
 (segment (start 107.696 46.5328) (end 107.696 53.1368) (width 0.5) (layer "F.Cu") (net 4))
 (segment (start 127.1016 45.8216) (end 108.4072 45.8216) (width 0.5) (layer "F.Cu") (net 4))
 (segment (start 105.7656 55.0672) (end 105.7656 55.118) (width 0.5) (layer "F.Cu") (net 4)))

